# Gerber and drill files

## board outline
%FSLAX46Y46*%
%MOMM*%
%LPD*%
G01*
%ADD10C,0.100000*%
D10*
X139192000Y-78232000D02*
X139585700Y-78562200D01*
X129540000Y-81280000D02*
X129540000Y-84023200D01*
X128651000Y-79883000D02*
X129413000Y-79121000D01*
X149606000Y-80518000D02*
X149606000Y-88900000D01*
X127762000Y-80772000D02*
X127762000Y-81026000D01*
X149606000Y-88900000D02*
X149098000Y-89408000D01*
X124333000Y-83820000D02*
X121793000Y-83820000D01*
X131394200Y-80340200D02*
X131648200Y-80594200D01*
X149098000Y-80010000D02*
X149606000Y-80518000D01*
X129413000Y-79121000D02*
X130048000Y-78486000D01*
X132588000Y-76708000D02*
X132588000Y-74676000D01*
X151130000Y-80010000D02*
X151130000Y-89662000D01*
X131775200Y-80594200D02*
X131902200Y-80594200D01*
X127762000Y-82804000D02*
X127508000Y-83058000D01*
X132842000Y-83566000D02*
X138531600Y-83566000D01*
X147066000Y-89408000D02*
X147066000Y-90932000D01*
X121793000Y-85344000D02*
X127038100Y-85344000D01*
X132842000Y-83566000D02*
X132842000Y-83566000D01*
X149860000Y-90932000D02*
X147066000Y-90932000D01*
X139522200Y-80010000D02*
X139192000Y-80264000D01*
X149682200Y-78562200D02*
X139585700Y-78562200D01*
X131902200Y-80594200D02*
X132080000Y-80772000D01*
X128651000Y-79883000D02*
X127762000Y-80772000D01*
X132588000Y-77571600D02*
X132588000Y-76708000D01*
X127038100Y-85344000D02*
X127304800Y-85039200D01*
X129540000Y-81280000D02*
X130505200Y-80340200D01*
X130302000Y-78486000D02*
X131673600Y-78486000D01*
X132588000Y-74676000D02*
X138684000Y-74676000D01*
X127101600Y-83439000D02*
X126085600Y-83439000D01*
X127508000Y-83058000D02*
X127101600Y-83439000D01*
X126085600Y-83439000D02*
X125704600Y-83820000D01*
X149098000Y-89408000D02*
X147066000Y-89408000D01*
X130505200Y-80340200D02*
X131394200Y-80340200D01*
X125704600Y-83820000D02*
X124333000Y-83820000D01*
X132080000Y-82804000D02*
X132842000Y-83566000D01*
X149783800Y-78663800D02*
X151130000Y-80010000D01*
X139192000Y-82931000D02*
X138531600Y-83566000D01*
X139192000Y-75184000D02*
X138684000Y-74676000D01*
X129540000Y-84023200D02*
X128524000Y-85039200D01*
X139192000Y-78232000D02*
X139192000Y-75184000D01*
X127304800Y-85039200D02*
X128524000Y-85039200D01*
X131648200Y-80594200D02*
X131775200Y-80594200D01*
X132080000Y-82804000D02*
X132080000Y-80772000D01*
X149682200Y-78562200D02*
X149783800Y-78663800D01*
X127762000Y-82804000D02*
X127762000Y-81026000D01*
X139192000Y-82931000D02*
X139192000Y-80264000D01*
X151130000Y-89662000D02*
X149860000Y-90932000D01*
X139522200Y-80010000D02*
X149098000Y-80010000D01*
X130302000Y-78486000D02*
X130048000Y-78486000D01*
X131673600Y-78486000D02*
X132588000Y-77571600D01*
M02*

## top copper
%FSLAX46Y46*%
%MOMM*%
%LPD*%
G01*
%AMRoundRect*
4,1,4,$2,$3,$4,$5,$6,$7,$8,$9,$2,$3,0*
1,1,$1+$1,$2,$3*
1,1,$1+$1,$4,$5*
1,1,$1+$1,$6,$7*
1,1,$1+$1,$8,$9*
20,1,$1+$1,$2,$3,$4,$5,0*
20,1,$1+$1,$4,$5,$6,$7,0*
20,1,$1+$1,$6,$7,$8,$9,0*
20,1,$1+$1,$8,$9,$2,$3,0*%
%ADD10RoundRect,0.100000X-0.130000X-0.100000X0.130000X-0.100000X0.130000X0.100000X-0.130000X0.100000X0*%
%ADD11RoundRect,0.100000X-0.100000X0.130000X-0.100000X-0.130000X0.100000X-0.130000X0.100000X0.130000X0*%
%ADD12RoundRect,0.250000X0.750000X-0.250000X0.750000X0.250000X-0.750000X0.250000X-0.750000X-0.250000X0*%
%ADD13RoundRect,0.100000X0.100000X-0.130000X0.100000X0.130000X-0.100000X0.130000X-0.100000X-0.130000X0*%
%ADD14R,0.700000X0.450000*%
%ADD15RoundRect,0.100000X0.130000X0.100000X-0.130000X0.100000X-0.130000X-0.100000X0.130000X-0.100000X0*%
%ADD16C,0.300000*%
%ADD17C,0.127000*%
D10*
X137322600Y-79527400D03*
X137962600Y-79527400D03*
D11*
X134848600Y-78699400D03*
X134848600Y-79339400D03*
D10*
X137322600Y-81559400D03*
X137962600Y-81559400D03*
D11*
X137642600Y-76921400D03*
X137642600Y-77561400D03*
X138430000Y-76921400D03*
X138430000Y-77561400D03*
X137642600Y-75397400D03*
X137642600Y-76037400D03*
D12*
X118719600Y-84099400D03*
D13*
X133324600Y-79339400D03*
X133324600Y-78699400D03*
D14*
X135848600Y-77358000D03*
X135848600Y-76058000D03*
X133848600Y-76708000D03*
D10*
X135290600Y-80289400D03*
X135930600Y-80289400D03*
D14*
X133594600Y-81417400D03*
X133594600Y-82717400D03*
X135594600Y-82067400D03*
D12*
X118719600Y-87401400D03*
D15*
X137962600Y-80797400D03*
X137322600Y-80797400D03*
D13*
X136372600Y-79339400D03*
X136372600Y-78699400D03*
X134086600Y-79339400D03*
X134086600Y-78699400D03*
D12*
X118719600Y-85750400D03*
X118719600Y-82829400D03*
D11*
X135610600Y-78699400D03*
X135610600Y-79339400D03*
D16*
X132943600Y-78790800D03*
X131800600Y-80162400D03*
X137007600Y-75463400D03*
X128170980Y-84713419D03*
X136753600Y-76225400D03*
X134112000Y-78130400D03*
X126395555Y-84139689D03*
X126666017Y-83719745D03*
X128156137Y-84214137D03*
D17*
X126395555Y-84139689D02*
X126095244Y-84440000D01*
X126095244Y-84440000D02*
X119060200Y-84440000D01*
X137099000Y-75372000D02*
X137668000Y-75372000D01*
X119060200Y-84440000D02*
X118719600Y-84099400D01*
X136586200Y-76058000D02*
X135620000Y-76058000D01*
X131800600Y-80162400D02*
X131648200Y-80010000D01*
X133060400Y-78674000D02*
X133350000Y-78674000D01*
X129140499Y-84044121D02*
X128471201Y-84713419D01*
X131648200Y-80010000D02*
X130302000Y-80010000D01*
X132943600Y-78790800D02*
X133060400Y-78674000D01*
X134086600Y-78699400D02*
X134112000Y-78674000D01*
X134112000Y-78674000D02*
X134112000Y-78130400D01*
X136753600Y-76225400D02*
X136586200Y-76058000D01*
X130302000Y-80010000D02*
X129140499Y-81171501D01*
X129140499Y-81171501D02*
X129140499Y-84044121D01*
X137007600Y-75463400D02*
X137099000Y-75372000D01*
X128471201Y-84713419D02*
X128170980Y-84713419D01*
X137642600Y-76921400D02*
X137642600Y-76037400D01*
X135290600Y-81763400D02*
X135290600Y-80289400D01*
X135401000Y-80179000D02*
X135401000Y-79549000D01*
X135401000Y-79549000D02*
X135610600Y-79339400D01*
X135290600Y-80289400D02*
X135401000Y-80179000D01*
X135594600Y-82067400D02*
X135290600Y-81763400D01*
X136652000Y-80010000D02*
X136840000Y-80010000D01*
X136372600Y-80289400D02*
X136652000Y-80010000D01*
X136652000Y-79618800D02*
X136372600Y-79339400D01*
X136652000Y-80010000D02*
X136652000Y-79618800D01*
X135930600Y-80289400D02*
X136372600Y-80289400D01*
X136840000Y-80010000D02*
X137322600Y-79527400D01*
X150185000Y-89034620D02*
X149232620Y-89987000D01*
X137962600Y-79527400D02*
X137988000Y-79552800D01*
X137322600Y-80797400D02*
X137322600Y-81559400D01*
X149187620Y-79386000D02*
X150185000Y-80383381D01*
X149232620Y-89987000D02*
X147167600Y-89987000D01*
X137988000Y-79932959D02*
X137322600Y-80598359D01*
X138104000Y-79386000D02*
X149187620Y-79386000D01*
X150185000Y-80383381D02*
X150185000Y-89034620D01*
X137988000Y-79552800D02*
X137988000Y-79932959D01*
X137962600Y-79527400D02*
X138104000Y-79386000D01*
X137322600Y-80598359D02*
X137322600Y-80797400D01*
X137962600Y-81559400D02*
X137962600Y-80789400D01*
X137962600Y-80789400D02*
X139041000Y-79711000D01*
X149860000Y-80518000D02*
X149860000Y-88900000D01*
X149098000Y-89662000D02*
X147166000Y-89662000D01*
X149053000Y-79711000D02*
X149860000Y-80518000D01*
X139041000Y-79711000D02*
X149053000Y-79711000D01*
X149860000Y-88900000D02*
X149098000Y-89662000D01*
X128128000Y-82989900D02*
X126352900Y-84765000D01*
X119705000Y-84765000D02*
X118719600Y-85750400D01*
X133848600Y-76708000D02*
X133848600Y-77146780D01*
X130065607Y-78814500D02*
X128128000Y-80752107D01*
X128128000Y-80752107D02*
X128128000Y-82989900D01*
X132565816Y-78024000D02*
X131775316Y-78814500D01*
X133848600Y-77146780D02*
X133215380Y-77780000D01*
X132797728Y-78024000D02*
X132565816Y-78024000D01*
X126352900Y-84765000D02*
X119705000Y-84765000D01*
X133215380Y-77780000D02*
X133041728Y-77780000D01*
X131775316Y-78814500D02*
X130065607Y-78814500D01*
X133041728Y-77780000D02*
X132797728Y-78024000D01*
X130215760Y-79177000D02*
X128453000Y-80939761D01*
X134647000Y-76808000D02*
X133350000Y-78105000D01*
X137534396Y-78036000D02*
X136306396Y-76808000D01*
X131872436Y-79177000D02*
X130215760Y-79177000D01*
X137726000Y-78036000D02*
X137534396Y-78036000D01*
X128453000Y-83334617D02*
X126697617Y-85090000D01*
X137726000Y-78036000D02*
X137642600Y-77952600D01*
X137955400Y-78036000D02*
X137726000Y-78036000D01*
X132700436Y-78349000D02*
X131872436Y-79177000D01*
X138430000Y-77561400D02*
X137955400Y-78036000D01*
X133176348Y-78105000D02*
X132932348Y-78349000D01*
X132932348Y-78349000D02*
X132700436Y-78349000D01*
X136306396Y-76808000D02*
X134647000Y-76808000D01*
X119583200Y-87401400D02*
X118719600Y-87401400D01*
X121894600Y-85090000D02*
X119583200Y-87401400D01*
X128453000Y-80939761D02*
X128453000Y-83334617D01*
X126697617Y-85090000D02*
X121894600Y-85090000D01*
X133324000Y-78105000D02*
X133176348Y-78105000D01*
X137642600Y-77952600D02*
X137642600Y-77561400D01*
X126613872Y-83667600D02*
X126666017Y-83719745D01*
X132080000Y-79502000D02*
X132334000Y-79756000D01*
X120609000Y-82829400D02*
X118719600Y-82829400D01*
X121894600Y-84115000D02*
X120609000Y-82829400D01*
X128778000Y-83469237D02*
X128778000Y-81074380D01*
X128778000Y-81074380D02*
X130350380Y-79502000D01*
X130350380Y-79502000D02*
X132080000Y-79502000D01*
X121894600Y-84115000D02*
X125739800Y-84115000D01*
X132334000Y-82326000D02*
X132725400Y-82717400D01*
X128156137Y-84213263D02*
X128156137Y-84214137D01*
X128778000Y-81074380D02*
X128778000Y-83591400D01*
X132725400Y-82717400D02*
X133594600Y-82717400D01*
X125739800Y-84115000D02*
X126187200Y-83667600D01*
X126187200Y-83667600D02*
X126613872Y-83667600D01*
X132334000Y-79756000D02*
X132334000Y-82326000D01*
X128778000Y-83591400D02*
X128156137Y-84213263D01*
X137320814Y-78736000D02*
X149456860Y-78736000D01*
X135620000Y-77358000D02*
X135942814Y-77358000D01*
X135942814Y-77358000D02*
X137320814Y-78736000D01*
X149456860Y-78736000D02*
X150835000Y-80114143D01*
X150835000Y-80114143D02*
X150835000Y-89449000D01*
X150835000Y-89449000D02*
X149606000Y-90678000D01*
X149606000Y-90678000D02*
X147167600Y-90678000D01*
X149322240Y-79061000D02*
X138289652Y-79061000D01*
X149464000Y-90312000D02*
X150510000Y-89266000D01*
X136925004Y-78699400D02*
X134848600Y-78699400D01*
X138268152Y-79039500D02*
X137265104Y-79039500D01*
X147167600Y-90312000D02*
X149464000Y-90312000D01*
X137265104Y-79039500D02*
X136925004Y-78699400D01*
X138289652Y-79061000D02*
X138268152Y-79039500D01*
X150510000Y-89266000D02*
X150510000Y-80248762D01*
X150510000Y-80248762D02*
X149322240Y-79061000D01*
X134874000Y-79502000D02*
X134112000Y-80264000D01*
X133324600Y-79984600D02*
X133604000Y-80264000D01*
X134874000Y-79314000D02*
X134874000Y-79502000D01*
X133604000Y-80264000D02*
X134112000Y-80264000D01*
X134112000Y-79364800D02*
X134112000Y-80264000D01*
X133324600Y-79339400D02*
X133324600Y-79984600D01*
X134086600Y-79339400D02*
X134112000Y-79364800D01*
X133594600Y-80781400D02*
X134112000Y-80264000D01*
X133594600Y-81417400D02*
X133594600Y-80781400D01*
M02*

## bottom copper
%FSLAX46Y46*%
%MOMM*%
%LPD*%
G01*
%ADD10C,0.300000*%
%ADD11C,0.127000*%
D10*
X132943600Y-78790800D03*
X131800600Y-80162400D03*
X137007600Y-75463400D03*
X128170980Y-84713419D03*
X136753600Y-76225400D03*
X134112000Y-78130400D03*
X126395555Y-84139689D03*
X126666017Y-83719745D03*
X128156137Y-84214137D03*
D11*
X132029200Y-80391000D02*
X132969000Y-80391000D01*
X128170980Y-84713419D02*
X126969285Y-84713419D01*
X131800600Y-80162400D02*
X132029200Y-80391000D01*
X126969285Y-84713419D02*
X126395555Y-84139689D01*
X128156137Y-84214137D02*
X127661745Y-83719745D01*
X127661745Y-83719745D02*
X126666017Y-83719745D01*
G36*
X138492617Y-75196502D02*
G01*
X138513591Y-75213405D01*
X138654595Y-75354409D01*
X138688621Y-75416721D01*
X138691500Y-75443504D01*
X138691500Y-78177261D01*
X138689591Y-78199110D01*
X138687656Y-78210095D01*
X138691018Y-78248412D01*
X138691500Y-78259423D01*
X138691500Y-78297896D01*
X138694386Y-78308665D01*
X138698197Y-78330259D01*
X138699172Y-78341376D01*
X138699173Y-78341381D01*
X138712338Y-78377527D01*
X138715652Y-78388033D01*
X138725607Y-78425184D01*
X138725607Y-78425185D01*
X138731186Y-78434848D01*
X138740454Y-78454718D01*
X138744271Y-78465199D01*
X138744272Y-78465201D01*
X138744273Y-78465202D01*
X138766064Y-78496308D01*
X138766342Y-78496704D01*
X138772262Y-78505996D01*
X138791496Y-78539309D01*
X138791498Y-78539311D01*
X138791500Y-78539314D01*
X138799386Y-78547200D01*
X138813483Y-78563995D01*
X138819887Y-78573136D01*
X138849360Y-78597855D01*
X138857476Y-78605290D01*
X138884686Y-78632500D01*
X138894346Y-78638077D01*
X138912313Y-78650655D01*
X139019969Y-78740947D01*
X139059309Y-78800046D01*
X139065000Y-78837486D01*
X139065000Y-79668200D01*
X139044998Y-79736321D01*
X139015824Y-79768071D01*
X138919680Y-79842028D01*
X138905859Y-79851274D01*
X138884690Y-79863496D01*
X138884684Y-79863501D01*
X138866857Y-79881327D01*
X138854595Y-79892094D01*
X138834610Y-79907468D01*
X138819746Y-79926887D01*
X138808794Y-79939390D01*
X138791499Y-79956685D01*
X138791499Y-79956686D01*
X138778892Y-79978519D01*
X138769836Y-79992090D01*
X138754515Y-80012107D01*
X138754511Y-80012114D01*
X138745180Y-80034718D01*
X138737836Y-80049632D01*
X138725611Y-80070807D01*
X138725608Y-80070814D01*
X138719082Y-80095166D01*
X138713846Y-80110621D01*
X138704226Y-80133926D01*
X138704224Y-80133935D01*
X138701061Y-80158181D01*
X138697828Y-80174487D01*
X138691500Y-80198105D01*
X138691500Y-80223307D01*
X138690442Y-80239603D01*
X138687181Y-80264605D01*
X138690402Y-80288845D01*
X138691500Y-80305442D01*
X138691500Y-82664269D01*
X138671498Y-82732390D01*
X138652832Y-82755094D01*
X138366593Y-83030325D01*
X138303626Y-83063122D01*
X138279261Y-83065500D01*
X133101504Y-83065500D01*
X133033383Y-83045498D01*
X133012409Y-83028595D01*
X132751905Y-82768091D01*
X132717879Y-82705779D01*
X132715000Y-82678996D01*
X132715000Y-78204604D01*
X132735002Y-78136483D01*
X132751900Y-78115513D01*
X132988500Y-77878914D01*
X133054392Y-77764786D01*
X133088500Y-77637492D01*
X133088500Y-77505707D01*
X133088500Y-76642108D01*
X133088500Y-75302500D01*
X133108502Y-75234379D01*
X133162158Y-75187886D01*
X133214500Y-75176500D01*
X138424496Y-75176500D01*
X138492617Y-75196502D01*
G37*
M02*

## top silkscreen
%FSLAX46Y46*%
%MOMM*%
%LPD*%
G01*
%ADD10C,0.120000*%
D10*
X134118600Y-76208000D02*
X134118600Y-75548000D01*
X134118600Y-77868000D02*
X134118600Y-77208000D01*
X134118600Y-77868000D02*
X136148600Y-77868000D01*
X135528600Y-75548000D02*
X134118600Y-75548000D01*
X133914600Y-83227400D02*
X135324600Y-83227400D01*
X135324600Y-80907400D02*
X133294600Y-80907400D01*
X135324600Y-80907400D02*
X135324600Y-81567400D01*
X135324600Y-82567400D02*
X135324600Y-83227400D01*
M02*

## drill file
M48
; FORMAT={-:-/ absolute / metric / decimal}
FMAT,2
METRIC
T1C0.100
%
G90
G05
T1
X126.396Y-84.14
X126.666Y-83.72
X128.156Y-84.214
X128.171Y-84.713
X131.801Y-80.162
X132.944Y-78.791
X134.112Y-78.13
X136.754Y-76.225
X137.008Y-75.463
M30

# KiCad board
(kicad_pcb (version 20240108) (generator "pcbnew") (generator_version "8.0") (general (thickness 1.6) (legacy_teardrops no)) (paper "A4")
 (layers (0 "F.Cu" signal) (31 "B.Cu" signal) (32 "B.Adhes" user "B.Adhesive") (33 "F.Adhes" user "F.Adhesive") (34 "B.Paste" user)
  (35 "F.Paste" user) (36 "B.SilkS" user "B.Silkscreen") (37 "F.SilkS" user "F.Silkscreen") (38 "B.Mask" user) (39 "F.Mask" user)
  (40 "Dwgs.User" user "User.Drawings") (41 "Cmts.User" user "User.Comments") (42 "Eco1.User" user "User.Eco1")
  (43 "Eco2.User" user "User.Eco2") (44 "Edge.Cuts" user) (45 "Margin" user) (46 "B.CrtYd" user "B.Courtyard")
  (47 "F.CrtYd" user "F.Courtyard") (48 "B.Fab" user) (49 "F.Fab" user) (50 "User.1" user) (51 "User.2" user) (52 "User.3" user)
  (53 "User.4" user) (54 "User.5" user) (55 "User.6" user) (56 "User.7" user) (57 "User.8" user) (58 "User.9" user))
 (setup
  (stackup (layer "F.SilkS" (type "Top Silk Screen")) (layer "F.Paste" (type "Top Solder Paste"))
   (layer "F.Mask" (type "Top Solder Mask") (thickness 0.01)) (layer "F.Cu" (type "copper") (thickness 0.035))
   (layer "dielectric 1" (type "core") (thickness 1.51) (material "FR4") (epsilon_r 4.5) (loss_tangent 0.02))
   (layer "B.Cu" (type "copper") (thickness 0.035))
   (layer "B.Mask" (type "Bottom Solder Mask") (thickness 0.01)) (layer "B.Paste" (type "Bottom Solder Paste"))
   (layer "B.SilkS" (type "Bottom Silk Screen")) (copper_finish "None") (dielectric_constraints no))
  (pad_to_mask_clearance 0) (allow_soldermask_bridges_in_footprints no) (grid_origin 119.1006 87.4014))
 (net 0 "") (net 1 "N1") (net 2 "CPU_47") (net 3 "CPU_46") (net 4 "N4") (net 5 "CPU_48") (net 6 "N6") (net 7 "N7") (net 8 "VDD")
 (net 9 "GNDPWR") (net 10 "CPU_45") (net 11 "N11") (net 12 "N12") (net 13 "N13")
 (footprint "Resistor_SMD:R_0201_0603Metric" (layer "F.Cu") (at 137.6426 79.5274)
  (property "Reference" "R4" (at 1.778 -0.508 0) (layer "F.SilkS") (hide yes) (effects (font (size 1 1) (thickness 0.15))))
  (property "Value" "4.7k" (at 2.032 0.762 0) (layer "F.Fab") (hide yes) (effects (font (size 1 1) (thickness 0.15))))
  (pad "" smd roundrect (at -0.345 0) (size 0.318 0.36) (layers "F.Paste") (roundrect_rratio 0.25))
  (pad "" smd roundrect (at 0.345 0) (size 0.318 0.36) (layers "F.Paste") (roundrect_rratio 0.25))
  (pad "1" smd roundrect (at -0.32 0) (size 0.46 0.4) (layers "F.Cu" "F.Mask") (roundrect_rratio 0.25) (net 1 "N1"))
  (pad "2" smd roundrect (at 0.32 0) (size 0.46 0.4) (layers "F.Cu" "F.Mask") (roundrect_rratio 0.25) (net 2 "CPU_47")))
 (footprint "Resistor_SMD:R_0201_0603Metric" (layer "F.Cu") (at 134.8486 79.0194 -90)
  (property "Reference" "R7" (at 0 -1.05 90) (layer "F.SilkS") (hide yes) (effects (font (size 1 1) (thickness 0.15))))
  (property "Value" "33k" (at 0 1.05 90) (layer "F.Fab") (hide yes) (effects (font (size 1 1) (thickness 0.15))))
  (pad "" smd roundrect (at -0.345 0 270) (size 0.318 0.36) (layers "F.Paste") (roundrect_rratio 0.25))
  (pad "" smd roundrect (at 0.345 0 270) (size 0.318 0.36) (layers "F.Paste") (roundrect_rratio 0.25))
  (pad "1" smd roundrect (at -0.32 0 270) (size 0.46 0.4) (layers "F.Cu" "F.Mask") (roundrect_rratio 0.25) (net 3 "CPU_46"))
  (pad "2" smd roundrect (at 0.32 0 270) (size 0.46 0.4) (layers "F.Cu" "F.Mask") (roundrect_rratio 0.25) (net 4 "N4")))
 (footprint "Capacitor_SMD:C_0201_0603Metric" (layer "F.Cu") (at 137.6426 81.5594)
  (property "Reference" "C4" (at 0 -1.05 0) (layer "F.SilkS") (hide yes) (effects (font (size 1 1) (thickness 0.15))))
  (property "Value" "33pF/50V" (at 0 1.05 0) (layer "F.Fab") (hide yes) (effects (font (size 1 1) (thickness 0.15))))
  (pad "" smd roundrect (at -0.345 0) (size 0.318 0.36) (layers "F.Paste") (roundrect_rratio 0.25))
  (pad "" smd roundrect (at 0.345 0) (size 0.318 0.36) (layers "F.Paste") (roundrect_rratio 0.25))
  (pad "1" smd roundrect (at -0.32 0) (size 0.46 0.4) (layers "F.Cu" "F.Mask") (roundrect_rratio 0.25) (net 2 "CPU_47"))
  (pad "2" smd roundrect (at 0.32 0) (size 0.46 0.4) (layers "F.Cu" "F.Mask") (roundrect_rratio 0.25) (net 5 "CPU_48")))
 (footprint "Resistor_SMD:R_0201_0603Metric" (layer "F.Cu") (at 137.6426 77.2414 -90)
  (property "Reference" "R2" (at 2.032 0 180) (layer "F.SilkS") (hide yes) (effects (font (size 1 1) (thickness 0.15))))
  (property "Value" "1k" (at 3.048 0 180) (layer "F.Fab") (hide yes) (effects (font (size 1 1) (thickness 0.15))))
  (pad "" smd roundrect (at -0.345 0 270) (size 0.318 0.36) (layers "F.Paste") (roundrect_rratio 0.25))
  (pad "" smd roundrect (at 0.345 0 270) (size 0.318 0.36) (layers "F.Paste") (roundrect_rratio 0.25))
  (pad "1" smd roundrect (at -0.32 0 270) (size 0.46 0.4) (layers "F.Cu" "F.Mask") (roundrect_rratio 0.25) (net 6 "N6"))
  (pad "2" smd roundrect (at 0.32 0 270) (size 0.46 0.4) (layers "F.Cu" "F.Mask") (roundrect_rratio 0.25) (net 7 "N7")))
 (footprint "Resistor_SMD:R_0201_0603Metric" (layer "F.Cu") (at 138.43 77.2414 -90)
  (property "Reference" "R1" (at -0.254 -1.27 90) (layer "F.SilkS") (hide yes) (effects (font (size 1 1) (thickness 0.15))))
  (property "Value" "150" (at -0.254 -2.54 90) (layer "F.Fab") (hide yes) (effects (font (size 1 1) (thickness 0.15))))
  (pad "" smd roundrect (at -0.345 0 270) (size 0.318 0.36) (layers "F.Paste") (roundrect_rratio 0.25))
  (pad "" smd roundrect (at 0.345 0 270) (size 0.318 0.36) (layers "F.Paste") (roundrect_rratio 0.25))
  (pad "1" smd roundrect (at -0.32 0 270) (size 0.46 0.4) (layers "F.Cu" "F.Mask") (roundrect_rratio 0.25) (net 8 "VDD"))
  (pad "2" smd roundrect (at 0.32 0 270) (size 0.46 0.4) (layers "F.Cu" "F.Mask") (roundrect_rratio 0.25) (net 7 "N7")))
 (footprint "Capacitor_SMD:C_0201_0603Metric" (layer "F.Cu") (at 137.6426 75.7174 -90)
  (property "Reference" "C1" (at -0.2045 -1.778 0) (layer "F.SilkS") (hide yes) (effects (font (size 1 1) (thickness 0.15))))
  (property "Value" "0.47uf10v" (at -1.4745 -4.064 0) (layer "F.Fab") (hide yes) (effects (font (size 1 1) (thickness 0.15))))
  (pad "" smd roundrect (at -0.345 0 270) (size 0.318 0.36) (layers "F.Paste") (roundrect_rratio 0.25))
  (pad "" smd roundrect (at 0.345 0 270) (size 0.318 0.36) (layers "F.Paste") (roundrect_rratio 0.25))
  (pad "1" smd roundrect (at -0.32 0 270) (size 0.46 0.4) (layers "F.Cu" "F.Mask") (roundrect_rratio 0.25) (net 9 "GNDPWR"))
  (pad "2" smd roundrect (at 0.32 0 270) (size 0.46 0.4) (layers "F.Cu" "F.Mask") (roundrect_rratio 0.25) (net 6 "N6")))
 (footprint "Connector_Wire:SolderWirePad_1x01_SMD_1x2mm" (layer "F.Cu") (at 118.7196 84.0994 90)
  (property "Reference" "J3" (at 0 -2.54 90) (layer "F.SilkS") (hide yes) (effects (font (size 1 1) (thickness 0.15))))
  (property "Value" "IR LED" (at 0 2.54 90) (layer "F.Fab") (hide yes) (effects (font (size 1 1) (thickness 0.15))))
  (pad "1" smd roundrect (at 0 0 90) (size 1 2) (layers "F.Cu" "F.Paste" "F.Mask") (roundrect_rratio 0.25) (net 9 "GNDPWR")))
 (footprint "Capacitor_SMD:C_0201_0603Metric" (layer "F.Cu") (at 133.3246 79.0194 90)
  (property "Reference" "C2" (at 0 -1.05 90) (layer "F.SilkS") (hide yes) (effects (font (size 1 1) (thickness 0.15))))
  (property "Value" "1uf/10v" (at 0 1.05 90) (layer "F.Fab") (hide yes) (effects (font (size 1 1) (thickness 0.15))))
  (pad "" smd roundrect (at -0.345 0 90) (size 0.318 0.36) (layers "F.Paste") (roundrect_rratio 0.25))
  (pad "" smd roundrect (at 0.345 0 90) (size 0.318 0.36) (layers "F.Paste") (roundrect_rratio 0.25))
  (pad "1" smd roundrect (at -0.32 0 90) (size 0.46 0.4) (layers "F.Cu" "F.Mask") (roundrect_rratio 0.25) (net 4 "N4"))
  (pad "2" smd roundrect (at 0.32 0 90) (size 0.46 0.4) (layers "F.Cu" "F.Mask") (roundrect_rratio 0.25) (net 9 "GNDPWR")))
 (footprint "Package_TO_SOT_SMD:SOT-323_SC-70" (layer "F.Cu") (at 134.8486 76.708 180)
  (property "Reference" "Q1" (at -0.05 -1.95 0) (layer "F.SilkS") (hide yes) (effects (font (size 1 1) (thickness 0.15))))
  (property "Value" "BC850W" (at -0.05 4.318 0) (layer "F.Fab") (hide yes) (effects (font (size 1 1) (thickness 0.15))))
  (fp_line (start 0.73 0.5) (end 0.73 1.16) (stroke (width 0.12) (type solid)) (layer "F.SilkS"))
  (fp_line (start 0.73 -1.16) (end 0.73 -0.5) (stroke (width 0.12) (type solid)) (layer "F.SilkS"))
  (fp_line (start 0.73 -1.16) (end -1.3 -1.16) (stroke (width 0.12) (type solid)) (layer "F.SilkS"))
  (fp_line (start -0.68 1.16) (end 0.73 1.16) (stroke (width 0.12) (type solid)) (layer "F.SilkS"))
  (pad "1" smd rect (at -1 -0.65 90) (size 0.45 0.7) (layers "F.Cu" "F.Paste" "F.Mask") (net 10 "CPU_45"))
  (pad "2" smd rect (at -1 0.65 90) (size 0.45 0.7) (layers "F.Cu" "F.Paste" "F.Mask") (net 9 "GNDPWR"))
  (pad "3" smd rect (at 1 0 90) (size 0.45 0.7) (layers "F.Cu" "F.Paste" "F.Mask") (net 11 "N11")))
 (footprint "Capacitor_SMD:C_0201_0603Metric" (layer "F.Cu") (at 135.6106 80.2894)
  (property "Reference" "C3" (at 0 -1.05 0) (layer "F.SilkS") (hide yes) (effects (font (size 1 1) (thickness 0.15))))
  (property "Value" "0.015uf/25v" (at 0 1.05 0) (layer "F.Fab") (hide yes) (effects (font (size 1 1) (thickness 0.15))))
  (pad "" smd roundrect (at -0.345 0) (size 0.318 0.36) (layers "F.Paste") (roundrect_rratio 0.25))
  (pad "" smd roundrect (at 0.345 0) (size 0.318 0.36) (layers "F.Paste") (roundrect_rratio 0.25))
  (pad "1" smd roundrect (at -0.32 0) (size 0.46 0.4) (layers "F.Cu" "F.Mask") (roundrect_rratio 0.25) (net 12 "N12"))
  (pad "2" smd roundrect (at 0.32 0) (size 0.46 0.4) (layers "F.Cu" "F.Mask") (roundrect_rratio 0.25) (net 1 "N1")))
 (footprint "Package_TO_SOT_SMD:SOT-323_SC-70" (layer "F.Cu") (at 134.5946 82.0674)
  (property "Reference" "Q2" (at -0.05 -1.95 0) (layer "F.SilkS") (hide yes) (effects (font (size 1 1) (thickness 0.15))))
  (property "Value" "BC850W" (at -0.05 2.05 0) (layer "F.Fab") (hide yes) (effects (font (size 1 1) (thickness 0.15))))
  (fp_line (start -0.68 1.16) (end 0.73 1.16) (stroke (width 0.12) (type solid)) (layer "F.SilkS"))
  (fp_line (start 0.73 -1.16) (end -1.3 -1.16) (stroke (width 0.12) (type solid)) (layer "F.SilkS"))
  (fp_line (start 0.73 -1.16) (end 0.73 -0.5) (stroke (width 0.12) (type solid)) (layer "F.SilkS"))
  (fp_line (start 0.73 0.5) (end 0.73 1.16) (stroke (width 0.12) (type solid)) (layer "F.SilkS"))
  (pad "1" smd rect (at -1 -0.65 270) (size 0.45 0.7) (layers "F.Cu" "F.Paste" "F.Mask") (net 4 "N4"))
  (pad "2" smd rect (at -1 0.65 270) (size 0.45 0.7) (layers "F.Cu" "F.Paste" "F.Mask") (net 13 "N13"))
  (pad "3" smd rect (at 1 0 270) (size 0.45 0.7) (layers "F.Cu" "F.Paste" "F.Mask") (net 12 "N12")))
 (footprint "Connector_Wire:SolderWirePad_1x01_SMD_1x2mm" (layer "F.Cu") (at 118.7196 87.4014 90)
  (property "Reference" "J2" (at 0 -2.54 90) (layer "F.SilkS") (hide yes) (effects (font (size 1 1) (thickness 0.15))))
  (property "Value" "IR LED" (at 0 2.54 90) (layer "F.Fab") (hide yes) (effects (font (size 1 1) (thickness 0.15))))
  (pad "1" smd roundrect (at 0 0 90) (size 1 2) (layers "F.Cu" "F.Paste" "F.Mask") (roundrect_rratio 0.25) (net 7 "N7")))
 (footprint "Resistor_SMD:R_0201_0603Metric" (layer "F.Cu") (at 137.6426 80.7974 180)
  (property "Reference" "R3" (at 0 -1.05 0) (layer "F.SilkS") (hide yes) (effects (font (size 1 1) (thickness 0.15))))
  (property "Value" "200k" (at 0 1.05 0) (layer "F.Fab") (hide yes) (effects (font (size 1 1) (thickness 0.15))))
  (pad "" smd roundrect (at -0.345 0 180) (size 0.318 0.36) (layers "F.Paste") (roundrect_rratio 0.25))
  (pad "" smd roundrect (at 0.345 0 180) (size 0.318 0.36) (layers "F.Paste") (roundrect_rratio 0.25))
  (pad "1" smd roundrect (at -0.32 0 180) (size 0.46 0.4) (layers "F.Cu" "F.Mask") (roundrect_rratio 0.25) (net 5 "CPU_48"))
  (pad "2" smd roundrect (at 0.32 0 180) (size 0.46 0.4) (layers "F.Cu" "F.Mask") (roundrect_rratio 0.25) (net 2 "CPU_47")))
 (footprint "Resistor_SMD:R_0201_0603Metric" (layer "F.Cu") (at 136.3726 79.0194 90)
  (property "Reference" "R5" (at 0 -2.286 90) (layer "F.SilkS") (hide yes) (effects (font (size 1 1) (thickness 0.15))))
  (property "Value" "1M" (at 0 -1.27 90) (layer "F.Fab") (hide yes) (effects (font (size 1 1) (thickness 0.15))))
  (pad "" smd roundrect (at -0.345 0 90) (size 0.318 0.36) (layers "F.Paste") (roundrect_rratio 0.25))
  (pad "" smd roundrect (at 0.345 0 90) (size 0.318 0.36) (layers "F.Paste") (roundrect_rratio 0.25))
  (pad "1" smd roundrect (at -0.32 0 90) (size 0.46 0.4) (layers "F.Cu" "F.Mask") (roundrect_rratio 0.25) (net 1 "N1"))
  (pad "2" smd roundrect (at 0.32 0 90) (size 0.46 0.4) (layers "F.Cu" "F.Mask") (roundrect_rratio 0.25) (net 3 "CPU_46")))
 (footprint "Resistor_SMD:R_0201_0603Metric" (layer "F.Cu") (at 134.0866 79.0194 90)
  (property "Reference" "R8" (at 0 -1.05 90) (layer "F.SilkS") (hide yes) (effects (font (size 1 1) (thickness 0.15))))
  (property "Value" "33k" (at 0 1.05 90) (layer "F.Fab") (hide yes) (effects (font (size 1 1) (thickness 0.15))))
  (pad "" smd roundrect (at -0.345 0 90) (size 0.318 0.36) (layers "F.Paste") (roundrect_rratio 0.25))
  (pad "" smd roundrect (at 0.345 0 90) (size 0.318 0.36) (layers "F.Paste") (roundrect_rratio 0.25))
  (pad "1" smd roundrect (at -0.32 0 90) (size 0.46 0.4) (layers "F.Cu" "F.Mask") (roundrect_rratio 0.25) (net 4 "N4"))
  (pad "2" smd roundrect (at 0.32 0 90) (size 0.46 0.4) (layers "F.Cu" "F.Mask") (roundrect_rratio 0.25) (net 9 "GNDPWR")))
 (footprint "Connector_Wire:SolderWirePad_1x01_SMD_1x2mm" (layer "F.Cu") (at 118.7196 85.7504 90)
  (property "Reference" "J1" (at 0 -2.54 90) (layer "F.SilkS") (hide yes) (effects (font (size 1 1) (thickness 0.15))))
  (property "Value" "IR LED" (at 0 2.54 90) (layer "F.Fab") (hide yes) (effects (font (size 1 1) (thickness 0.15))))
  (pad "1" smd roundrect (at 0 0 90) (size 1 2) (layers "F.Cu" "F.Paste" "F.Mask") (roundrect_rratio 0.25) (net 11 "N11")))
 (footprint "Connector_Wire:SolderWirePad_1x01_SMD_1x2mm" (layer "F.Cu") (at 118.7196 82.8294 90)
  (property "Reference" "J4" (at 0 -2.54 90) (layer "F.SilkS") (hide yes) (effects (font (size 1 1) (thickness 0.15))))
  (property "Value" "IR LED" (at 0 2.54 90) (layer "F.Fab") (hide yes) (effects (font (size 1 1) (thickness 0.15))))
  (pad "1" smd roundrect (at 0 0 90) (size 1 2) (layers "F.Cu" "F.Paste" "F.Mask") (roundrect_rratio 0.25) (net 13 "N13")))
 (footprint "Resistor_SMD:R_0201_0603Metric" (layer "F.Cu") (at 135.6106 79.0194 -90)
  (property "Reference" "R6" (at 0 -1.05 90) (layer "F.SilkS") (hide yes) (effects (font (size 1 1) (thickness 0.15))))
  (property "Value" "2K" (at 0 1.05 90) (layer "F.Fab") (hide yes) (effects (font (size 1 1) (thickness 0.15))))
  (pad "" smd roundrect (at -0.345 0 270) (size 0.318 0.36) (layers "F.Paste") (roundrect_rratio 0.25))
  (pad "" smd roundrect (at 0.345 0 270) (size 0.318 0.36) (layers "F.Paste") (roundrect_rratio 0.25))
  (pad "1" smd roundrect (at -0.32 0 270) (size 0.46 0.4) (layers "F.Cu" "F.Mask") (roundrect_rratio 0.25) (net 3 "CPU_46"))
  (pad "2" smd roundrect (at 0.32 0 270) (size 0.46 0.4) (layers "F.Cu" "F.Mask") (roundrect_rratio 0.25) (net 12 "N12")))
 (gr_line (start 139.192 78.232) (end 139.5857 78.5622) (stroke (width 0.1) (type solid)) (layer "Edge.Cuts"))
 (gr_line (start 129.54 81.28) (end 129.54 84.0232) (stroke (width 0.1) (type solid)) (layer "Edge.Cuts"))
 (gr_line (start 128.651 79.883) (end 129.413 79.121) (stroke (width 0.1) (type solid)) (layer "Edge.Cuts"))
 (gr_line (start 149.606 80.518) (end 149.606 88.9) (stroke (width 0.1) (type solid)) (layer "Edge.Cuts"))
 (gr_line (start 127.762 80.772) (end 127.762 81.026) (stroke (width 0.1) (type solid)) (layer "Edge.Cuts"))
 (gr_line (start 149.606 88.9) (end 149.098 89.408) (stroke (width 0.1) (type solid)) (layer "Edge.Cuts"))
 (gr_line (start 124.333 83.82) (end 121.793 83.82) (stroke (width 0.1) (type solid)) (layer "Edge.Cuts"))
 (gr_line (start 131.3942 80.3402) (end 131.6482 80.5942) (stroke (width 0.1) (type solid)) (layer "Edge.Cuts"))
 (gr_line (start 149.098 80.01) (end 149.606 80.518) (stroke (width 0.1) (type solid)) (layer "Edge.Cuts"))
 (gr_line (start 129.413 79.121) (end 130.048 78.486) (stroke (width 0.1) (type solid)) (layer "Edge.Cuts"))
 (gr_line (start 132.588 76.708) (end 132.588 74.676) (stroke (width 0.1) (type solid)) (layer "Edge.Cuts"))
 (gr_line (start 151.13 80.01) (end 151.13 89.662) (stroke (width 0.1) (type solid)) (layer "Edge.Cuts"))
 (gr_line (start 131.7752 80.5942) (end 131.9022 80.5942) (stroke (width 0.1) (type solid)) (layer "Edge.Cuts"))
 (gr_line (start 127.762 82.804) (end 127.508 83.058) (stroke (width 0.1) (type solid)) (layer "Edge.Cuts"))
 (gr_line (start 132.842 83.566) (end 138.5316 83.566) (stroke (width 0.1) (type solid)) (layer "Edge.Cuts"))
 (gr_line (start 147.066 89.408) (end 147.066 90.932) (stroke (width 0.1) (type solid)) (layer "Edge.Cuts"))
 (gr_line (start 121.793 85.344) (end 127.0381 85.344) (stroke (width 0.1) (type solid)) (layer "Edge.Cuts"))
 (gr_line (start 132.842 83.566) (end 132.842 83.566) (stroke (width 0.1) (type solid)) (layer "Edge.Cuts"))
 (gr_line (start 149.86 90.932) (end 147.066 90.932) (stroke (width 0.1) (type solid)) (layer "Edge.Cuts"))
 (gr_line (start 139.5222 80.01) (end 139.192 80.264) (stroke (width 0.1) (type solid)) (layer "Edge.Cuts"))
 (gr_line (start 149.6822 78.5622) (end 139.5857 78.5622) (stroke (width 0.1) (type solid)) (layer "Edge.Cuts"))
 (gr_line (start 131.9022 80.5942) (end 132.08 80.772) (stroke (width 0.1) (type solid)) (layer "Edge.Cuts"))
 (gr_line (start 128.651 79.883) (end 127.762 80.772) (stroke (width 0.1) (type solid)) (layer "Edge.Cuts"))
 (gr_line (start 132.588 77.5716) (end 132.588 76.708) (stroke (width 0.1) (type solid)) (layer "Edge.Cuts"))
 (gr_line (start 127.0381 85.344) (end 127.3048 85.0392) (stroke (width 0.1) (type solid)) (layer "Edge.Cuts"))
 (gr_line (start 129.54 81.28) (end 130.5052 80.3402) (stroke (width 0.1) (type solid)) (layer "Edge.Cuts"))
 (gr_line (start 130.302 78.486) (end 131.6736 78.486) (stroke (width 0.1) (type solid)) (layer "Edge.Cuts"))
 (gr_line (start 132.588 74.676) (end 138.684 74.676) (stroke (width 0.1) (type solid)) (layer "Edge.Cuts"))
 (gr_line (start 127.1016 83.439) (end 126.0856 83.439) (stroke (width 0.1) (type solid)) (layer "Edge.Cuts"))
 (gr_line (start 127.508 83.058) (end 127.1016 83.439) (stroke (width 0.1) (type solid)) (layer "Edge.Cuts"))
 (gr_line (start 126.0856 83.439) (end 125.7046 83.82) (stroke (width 0.1) (type solid)) (layer "Edge.Cuts"))
 (gr_line (start 149.098 89.408) (end 147.066 89.408) (stroke (width 0.1) (type solid)) (layer "Edge.Cuts"))
 (gr_line (start 130.5052 80.3402) (end 131.3942 80.3402) (stroke (width 0.1) (type solid)) (layer "Edge.Cuts"))
 (gr_line (start 125.7046 83.82) (end 124.333 83.82) (stroke (width 0.1) (type solid)) (layer "Edge.Cuts"))
 (gr_line (start 132.08 82.804) (end 132.842 83.566) (stroke (width 0.1) (type solid)) (layer "Edge.Cuts"))
 (gr_line (start 149.7838 78.6638) (end 151.13 80.01) (stroke (width 0.1) (type solid)) (layer "Edge.Cuts"))
 (gr_line (start 139.192 82.931) (end 138.5316 83.566) (stroke (width 0.1) (type solid)) (layer "Edge.Cuts"))
 (gr_line (start 139.192 75.184) (end 138.684 74.676) (stroke (width 0.1) (type solid)) (layer "Edge.Cuts"))
 (gr_line (start 129.54 84.0232) (end 128.524 85.0392) (stroke (width 0.1) (type solid)) (layer "Edge.Cuts"))
 (gr_line (start 139.192 78.232) (end 139.192 75.184) (stroke (width 0.1) (type solid)) (layer "Edge.Cuts"))
 (gr_line (start 127.3048 85.0392) (end 128.524 85.0392) (stroke (width 0.1) (type solid)) (layer "Edge.Cuts"))
 (gr_line (start 131.6482 80.5942) (end 131.7752 80.5942) (stroke (width 0.1) (type solid)) (layer "Edge.Cuts"))
 (gr_line (start 132.08 82.804) (end 132.08 80.772) (stroke (width 0.1) (type solid)) (layer "Edge.Cuts"))
 (gr_line (start 149.6822 78.5622) (end 149.7838 78.6638) (stroke (width 0.1) (type solid)) (layer "Edge.Cuts"))
 (gr_line (start 127.762 82.804) (end 127.762 81.026) (stroke (width 0.1) (type solid)) (layer "Edge.Cuts"))
 (gr_line (start 139.192 82.931) (end 139.192 80.264) (stroke (width 0.1) (type solid)) (layer "Edge.Cuts"))
 (gr_line (start 151.13 89.662) (end 149.86 90.932) (stroke (width 0.1) (type solid)) (layer "Edge.Cuts"))
 (gr_line (start 139.5222 80.01) (end 149.098 80.01) (stroke (width 0.1) (type solid)) (layer "Edge.Cuts"))
 (gr_line (start 130.302 78.486) (end 130.048 78.486) (stroke (width 0.1) (type solid)) (layer "Edge.Cuts"))
 (gr_line (start 131.6736 78.486) (end 132.588 77.5716) (stroke (width 0.1) (type solid)) (layer "Edge.Cuts"))
 (segment (start 126.395555 84.139689) (end 126.095244 84.44) (width 0.127) (layer "F.Cu") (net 9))
 (segment (start 126.095244 84.44) (end 119.0602 84.44) (width 0.127) (layer "F.Cu") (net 9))
 (segment (start 137.099 75.372) (end 137.668 75.372) (width 0.127) (layer "F.Cu") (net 9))
 (segment (start 119.0602 84.44) (end 118.7196 84.0994) (width 0.127) (layer "F.Cu") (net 9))
 (segment (start 136.5862 76.058) (end 135.62 76.058) (width 0.127) (layer "F.Cu") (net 9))
 (segment (start 131.8006 80.1624) (end 131.6482 80.01) (width 0.127) (layer "F.Cu") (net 9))
 (segment (start 133.0604 78.674) (end 133.35 78.674) (width 0.127) (layer "F.Cu") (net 9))
 (segment (start 129.140499 84.044121) (end 128.471201 84.713419) (width 0.127) (layer "F.Cu") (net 9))
 (segment (start 131.6482 80.01) (end 130.302 80.01) (width 0.127) (layer "F.Cu") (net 9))
 (segment (start 132.9436 78.7908) (end 133.0604 78.674) (width 0.127) (layer "F.Cu") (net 9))
 (segment (start 134.0866 78.6994) (end 134.112 78.674) (width 0.127) (layer "F.Cu") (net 9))
 (segment (start 134.112 78.674) (end 134.112 78.1304) (width 0.127) (layer "F.Cu") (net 9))
 (segment (start 136.7536 76.2254) (end 136.5862 76.058) (width 0.127) (layer "F.Cu") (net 9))
 (segment (start 130.302 80.01) (end 129.140499 81.171501) (width 0.127) (layer "F.Cu") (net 9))
 (segment (start 129.140499 81.171501) (end 129.140499 84.044121) (width 0.127) (layer "F.Cu") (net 9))
 (segment (start 137.0076 75.4634) (end 137.099 75.372) (width 0.127) (layer "F.Cu") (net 9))
 (segment (start 128.471201 84.713419) (end 128.17098 84.713419) (width 0.127) (layer "F.Cu") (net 9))
 (via micro (at 132.9436 78.7908) (size 0.3) (drill 0.1) (layers "F.Cu" "B.Cu") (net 9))
 (via micro (at 131.8006 80.1624) (size 0.3) (drill 0.1) (layers "F.Cu" "B.Cu") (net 9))
 (via micro (at 137.0076 75.4634) (size 0.3) (drill 0.1) (layers "F.Cu" "B.Cu") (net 9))
 (via micro (at 128.17098 84.713419) (size 0.3) (drill 0.1) (layers "F.Cu" "B.Cu") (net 9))
 (via micro (at 136.7536 76.2254) (size 0.3) (drill 0.1) (layers "F.Cu" "B.Cu") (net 9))
 (via micro (at 134.112 78.1304) (size 0.3) (drill 0.1) (layers "F.Cu" "B.Cu") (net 9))
 (via micro (at 126.395555 84.139689) (size 0.3) (drill 0.1) (layers "F.Cu" "B.Cu") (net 9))
 (segment (start 132.0292 80.391) (end 132.969 80.391) (width 0.127) (layer "B.Cu") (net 9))
 (segment (start 128.17098 84.713419) (end 126.969285 84.713419) (width 0.127) (layer "B.Cu") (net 9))
 (segment (start 131.8006 80.1624) (end 132.0292 80.391) (width 0.127) (layer "B.Cu") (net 9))
 (segment (start 126.969285 84.713419) (end 126.395555 84.139689) (width 0.127) (layer "B.Cu") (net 9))
 (segment (start 137.6426 76.9214) (end 137.6426 76.0374) (width 0.127) (layer "F.Cu") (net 6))
 (segment (start 135.2906 81.7634) (end 135.2906 80.2894) (width 0.127) (layer "F.Cu") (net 12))
 (segment (start 135.401 80.179) (end 135.401 79.549) (width 0.127) (layer "F.Cu") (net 12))
 (segment (start 135.401 79.549) (end 135.6106 79.3394) (width 0.127) (layer "F.Cu") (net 12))
 (segment (start 135.2906 80.2894) (end 135.401 80.179) (width 0.127) (layer "F.Cu") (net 12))
 (segment (start 135.5946 82.0674) (end 135.2906 81.7634) (width 0.127) (layer "F.Cu") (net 12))
 (segment (start 136.652 80.01) (end 136.84 80.01) (width 0.127) (layer "F.Cu") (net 1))
 (segment (start 136.3726 80.2894) (end 136.652 80.01) (width 0.127) (layer "F.Cu") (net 1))
 (segment (start 136.652 79.6188) (end 136.3726 79.3394) (width 0.127) (layer "F.Cu") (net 1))
 (segment (start 136.652 80.01) (end 136.652 79.6188) (width 0.127) (layer "F.Cu") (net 1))
 (segment (start 135.9306 80.2894) (end 136.3726 80.2894) (width 0.127) (layer "F.Cu") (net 1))
 (segment (start 136.84 80.01) (end 137.3226 79.5274) (width 0.127) (layer "F.Cu") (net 1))
 (segment (start 150.185 89.03462) (end 149.23262 89.987) (width 0.127) (layer "F.Cu") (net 2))
 (segment (start 137.9626 79.5274) (end 137.988 79.5528) (width 0.127) (layer "F.Cu") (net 2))
 (segment (start 137.3226 80.7974) (end 137.3226 81.5594) (width 0.127) (layer "F.Cu") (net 2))
 (segment (start 149.18762 79.386) (end 150.185 80.383381) (width 0.127) (layer "F.Cu") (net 2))
 (segment (start 149.23262 89.987) (end 147.1676 89.987) (width 0.127) (layer "F.Cu") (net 2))
 (segment (start 137.988 79.932959) (end 137.3226 80.598359) (width 0.127) (layer "F.Cu") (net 2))
 (segment (start 138.104 79.386) (end 149.18762 79.386) (width 0.127) (layer "F.Cu") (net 2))
 (segment (start 150.185 80.383381) (end 150.185 89.03462) (width 0.127) (layer "F.Cu") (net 2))
 (segment (start 137.988 79.5528) (end 137.988 79.932959) (width 0.127) (layer "F.Cu") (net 2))
 (segment (start 137.9626 79.5274) (end 138.104 79.386) (width 0.127) (layer "F.Cu") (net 2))
 (segment (start 137.3226 80.598359) (end 137.3226 80.7974) (width 0.127) (layer "F.Cu") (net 2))
 (segment (start 137.9626 81.5594) (end 137.9626 80.7894) (width 0.127) (layer "F.Cu") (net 5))
 (segment (start 137.9626 80.7894) (end 139.041 79.711) (width 0.127) (layer "F.Cu") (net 5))
 (segment (start 149.86 80.518) (end 149.86 88.9) (width 0.127) (layer "F.Cu") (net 5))
 (segment (start 149.098 89.662) (end 147.166 89.662) (width 0.127) (layer "F.Cu") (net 5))
 (segment (start 149.053 79.711) (end 149.86 80.518) (width 0.127) (layer "F.Cu") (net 5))
 (segment (start 139.041 79.711) (end 149.053 79.711) (width 0.127) (layer "F.Cu") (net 5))
 (segment (start 149.86 88.9) (end 149.098 89.662) (width 0.127) (layer "F.Cu") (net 5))
 (segment (start 128.128 82.9899) (end 126.3529 84.765) (width 0.127) (layer "F.Cu") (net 11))
 (segment (start 119.705 84.765) (end 118.7196 85.7504) (width 0.127) (layer "F.Cu") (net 11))
 (segment (start 133.8486 76.708) (end 133.8486 77.14678) (width 0.127) (layer "F.Cu") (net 11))
 (segment (start 130.065607 78.8145) (end 128.128 80.752107) (width 0.127) (layer "F.Cu") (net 11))
 (segment (start 128.128 80.752107) (end 128.128 82.9899) (width 0.127) (layer "F.Cu") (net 11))
 (segment (start 132.565816 78.024) (end 131.775316 78.8145) (width 0.127) (layer "F.Cu") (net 11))
 (segment (start 133.8486 77.14678) (end 133.21538 77.78) (width 0.127) (layer "F.Cu") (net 11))
 (segment (start 132.797728 78.024) (end 132.565816 78.024) (width 0.127) (layer "F.Cu") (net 11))
 (segment (start 126.3529 84.765) (end 119.705 84.765) (width 0.127) (layer "F.Cu") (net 11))
 (segment (start 133.21538 77.78) (end 133.041728 77.78) (width 0.127) (layer "F.Cu") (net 11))
 (segment (start 131.775316 78.8145) (end 130.065607 78.8145) (width 0.127) (layer "F.Cu") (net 11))
 (segment (start 133.041728 77.78) (end 132.797728 78.024) (width 0.127) (layer "F.Cu") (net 11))
 (segment (start 130.21576 79.177) (end 128.453 80.939761) (width 0.127) (layer "F.Cu") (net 7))
 (segment (start 134.647 76.808) (end 133.35 78.105) (width 0.127) (layer "F.Cu") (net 7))
 (segment (start 137.534396 78.036) (end 136.306396 76.808) (width 0.127) (layer "F.Cu") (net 7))
 (segment (start 131.872436 79.177) (end 130.21576 79.177) (width 0.127) (layer "F.Cu") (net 7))
 (segment (start 137.726 78.036) (end 137.534396 78.036) (width 0.127) (layer "F.Cu") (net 7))
 (segment (start 128.453 83.334617) (end 126.697617 85.09) (width 0.127) (layer "F.Cu") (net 7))
 (segment (start 137.726 78.036) (end 137.6426 77.9526) (width 0.127) (layer "F.Cu") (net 7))
 (segment (start 137.9554 78.036) (end 137.726 78.036) (width 0.127) (layer "F.Cu") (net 7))
 (segment (start 132.700436 78.349) (end 131.872436 79.177) (width 0.127) (layer "F.Cu") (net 7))
 (segment (start 138.43 77.5614) (end 137.9554 78.036) (width 0.127) (layer "F.Cu") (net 7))
 (segment (start 133.176348 78.105) (end 132.932348 78.349) (width 0.127) (layer "F.Cu") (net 7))
 (segment (start 132.932348 78.349) (end 132.700436 78.349) (width 0.127) (layer "F.Cu") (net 7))
 (segment (start 136.306396 76.808) (end 134.647 76.808) (width 0.127) (layer "F.Cu") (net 7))
 (segment (start 119.5832 87.4014) (end 118.7196 87.4014) (width 0.127) (layer "F.Cu") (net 7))
 (segment (start 121.8946 85.09) (end 119.5832 87.4014) (width 0.127) (layer "F.Cu") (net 7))
 (segment (start 128.453 80.939761) (end 128.453 83.334617) (width 0.127) (layer "F.Cu") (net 7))
 (segment (start 126.697617 85.09) (end 121.8946 85.09) (width 0.127) (layer "F.Cu") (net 7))
 (segment (start 133.324 78.105) (end 133.176348 78.105) (width 0.127) (layer "F.Cu") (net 7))
 (segment (start 137.6426 77.9526) (end 137.6426 77.5614) (width 0.127) (layer "F.Cu") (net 7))
 (segment (start 126.613872 83.6676) (end 126.666017 83.719745) (width 0.127) (layer "F.Cu") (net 13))
 (segment (start 132.08 79.502) (end 132.334 79.756) (width 0.127) (layer "F.Cu") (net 13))
 (segment (start 120.609 82.8294) (end 118.7196 82.8294) (width 0.127) (layer "F.Cu") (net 13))
 (segment (start 121.8946 84.115) (end 120.609 82.8294) (width 0.127) (layer "F.Cu") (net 13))
 (segment (start 128.778 83.469237) (end 128.778 81.07438) (width 0.127) (layer "F.Cu") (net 13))
 (segment (start 128.778 81.07438) (end 130.35038 79.502) (width 0.127) (layer "F.Cu") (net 13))
 (segment (start 130.35038 79.502) (end 132.08 79.502) (width 0.127) (layer "F.Cu") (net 13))
 (segment (start 121.8946 84.115) (end 125.7398 84.115) (width 0.127) (layer "F.Cu") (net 13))
 (segment (start 132.334 82.326) (end 132.7254 82.7174) (width 0.127) (layer "F.Cu") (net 13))
 (segment (start 128.156137 84.213263) (end 128.156137 84.214137) (width 0.127) (layer "F.Cu") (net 13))
 (segment (start 128.778 81.07438) (end 128.778 83.5914) (width 0.127) (layer "F.Cu") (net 13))
 (segment (start 132.7254 82.7174) (end 133.5946 82.7174) (width 0.127) (layer "F.Cu") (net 13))
 (segment (start 125.7398 84.115) (end 126.1872 83.6676) (width 0.127) (layer "F.Cu") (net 13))
 (segment (start 126.1872 83.6676) (end 126.613872 83.6676) (width 0.127) (layer "F.Cu") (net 13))
 (segment (start 132.334 79.756) (end 132.334 82.326) (width 0.127) (layer "F.Cu") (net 13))
 (segment (start 128.778 83.5914) (end 128.156137 84.213263) (width 0.127) (layer "F.Cu") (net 13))
 (via micro (at 126.666017 83.719745) (size 0.3) (drill 0.1) (layers "F.Cu" "B.Cu") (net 13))
 (via micro (at 128.156137 84.214137) (size 0.3) (drill 0.1) (layers "F.Cu" "B.Cu") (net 13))
 (segment (start 128.156137 84.214137) (end 127.661745 83.719745) (width 0.127) (layer "B.Cu") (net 13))
 (segment (start 127.661745 83.719745) (end 126.666017 83.719745) (width 0.127) (layer "B.Cu") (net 13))
 (segment (start 137.320814 78.736) (end 149.45686 78.736) (width 0.127) (layer "F.Cu") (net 10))
 (segment (start 135.62 77.358) (end 135.942814 77.358) (width 0.127) (layer "F.Cu") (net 10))
 (segment (start 135.942814 77.358) (end 137.320814 78.736) (width 0.127) (layer "F.Cu") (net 10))
 (segment (start 149.45686 78.736) (end 150.835 80.114143) (width 0.127) (layer "F.Cu") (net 10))
 (segment (start 150.835 80.114143) (end 150.835 89.449) (width 0.127) (layer "F.Cu") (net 10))
 (segment (start 150.835 89.449) (end 149.606 90.678) (width 0.127) (layer "F.Cu") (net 10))
 (segment (start 149.606 90.678) (end 147.1676 90.678) (width 0.127) (layer "F.Cu") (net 10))
 (segment (start 149.32224 79.061) (end 138.289652 79.061) (width 0.127) (layer "F.Cu") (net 3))
 (segment (start 149.464 90.312) (end 150.51 89.266) (width 0.127) (layer "F.Cu") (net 3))
 (segment (start 136.925004 78.6994) (end 134.8486 78.6994) (width 0.127) (layer "F.Cu") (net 3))
 (segment (start 138.268152 79.0395) (end 137.265104 79.0395) (width 0.127) (layer "F.Cu") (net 3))
 (segment (start 147.1676 90.312) (end 149.464 90.312) (width 0.127) (layer "F.Cu") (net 3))
 (segment (start 137.265104 79.0395) (end 136.925004 78.6994) (width 0.127) (layer "F.Cu") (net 3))
 (segment (start 138.289652 79.061) (end 138.268152 79.0395) (width 0.127) (layer "F.Cu") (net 3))
 (segment (start 150.51 89.266) (end 150.51 80.248762) (width 0.127) (layer "F.Cu") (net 3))
 (segment (start 150.51 80.248762) (end 149.32224 79.061) (width 0.127) (layer "F.Cu") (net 3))
 (segment (start 134.874 79.502) (end 134.112 80.264) (width 0.127) (layer "F.Cu") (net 4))
 (segment (start 133.3246 79.9846) (end 133.604 80.264) (width 0.127) (layer "F.Cu") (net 4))
 (segment (start 134.874 79.314) (end 134.874 79.502) (width 0.127) (layer "F.Cu") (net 4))
 (segment (start 133.604 80.264) (end 134.112 80.264) (width 0.127) (layer "F.Cu") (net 4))
 (segment (start 134.112 79.3648) (end 134.112 80.264) (width 0.127) (layer "F.Cu") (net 4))
 (segment (start 133.3246 79.3394) (end 133.3246 79.9846) (width 0.127) (layer "F.Cu") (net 4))
 (segment (start 134.0866 79.3394) (end 134.112 79.3648) (width 0.127) (layer "F.Cu") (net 4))
 (segment (start 133.5946 80.7814) (end 134.112 80.264) (width 0.127) (layer "F.Cu") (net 4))
 (segment (start 133.5946 81.4174) (end 133.5946 80.7814) (width 0.127) (layer "F.Cu") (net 4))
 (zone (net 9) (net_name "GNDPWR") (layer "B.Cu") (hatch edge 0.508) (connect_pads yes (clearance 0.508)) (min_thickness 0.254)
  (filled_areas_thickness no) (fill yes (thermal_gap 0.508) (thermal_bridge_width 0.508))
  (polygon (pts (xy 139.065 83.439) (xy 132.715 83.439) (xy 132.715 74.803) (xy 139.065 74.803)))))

